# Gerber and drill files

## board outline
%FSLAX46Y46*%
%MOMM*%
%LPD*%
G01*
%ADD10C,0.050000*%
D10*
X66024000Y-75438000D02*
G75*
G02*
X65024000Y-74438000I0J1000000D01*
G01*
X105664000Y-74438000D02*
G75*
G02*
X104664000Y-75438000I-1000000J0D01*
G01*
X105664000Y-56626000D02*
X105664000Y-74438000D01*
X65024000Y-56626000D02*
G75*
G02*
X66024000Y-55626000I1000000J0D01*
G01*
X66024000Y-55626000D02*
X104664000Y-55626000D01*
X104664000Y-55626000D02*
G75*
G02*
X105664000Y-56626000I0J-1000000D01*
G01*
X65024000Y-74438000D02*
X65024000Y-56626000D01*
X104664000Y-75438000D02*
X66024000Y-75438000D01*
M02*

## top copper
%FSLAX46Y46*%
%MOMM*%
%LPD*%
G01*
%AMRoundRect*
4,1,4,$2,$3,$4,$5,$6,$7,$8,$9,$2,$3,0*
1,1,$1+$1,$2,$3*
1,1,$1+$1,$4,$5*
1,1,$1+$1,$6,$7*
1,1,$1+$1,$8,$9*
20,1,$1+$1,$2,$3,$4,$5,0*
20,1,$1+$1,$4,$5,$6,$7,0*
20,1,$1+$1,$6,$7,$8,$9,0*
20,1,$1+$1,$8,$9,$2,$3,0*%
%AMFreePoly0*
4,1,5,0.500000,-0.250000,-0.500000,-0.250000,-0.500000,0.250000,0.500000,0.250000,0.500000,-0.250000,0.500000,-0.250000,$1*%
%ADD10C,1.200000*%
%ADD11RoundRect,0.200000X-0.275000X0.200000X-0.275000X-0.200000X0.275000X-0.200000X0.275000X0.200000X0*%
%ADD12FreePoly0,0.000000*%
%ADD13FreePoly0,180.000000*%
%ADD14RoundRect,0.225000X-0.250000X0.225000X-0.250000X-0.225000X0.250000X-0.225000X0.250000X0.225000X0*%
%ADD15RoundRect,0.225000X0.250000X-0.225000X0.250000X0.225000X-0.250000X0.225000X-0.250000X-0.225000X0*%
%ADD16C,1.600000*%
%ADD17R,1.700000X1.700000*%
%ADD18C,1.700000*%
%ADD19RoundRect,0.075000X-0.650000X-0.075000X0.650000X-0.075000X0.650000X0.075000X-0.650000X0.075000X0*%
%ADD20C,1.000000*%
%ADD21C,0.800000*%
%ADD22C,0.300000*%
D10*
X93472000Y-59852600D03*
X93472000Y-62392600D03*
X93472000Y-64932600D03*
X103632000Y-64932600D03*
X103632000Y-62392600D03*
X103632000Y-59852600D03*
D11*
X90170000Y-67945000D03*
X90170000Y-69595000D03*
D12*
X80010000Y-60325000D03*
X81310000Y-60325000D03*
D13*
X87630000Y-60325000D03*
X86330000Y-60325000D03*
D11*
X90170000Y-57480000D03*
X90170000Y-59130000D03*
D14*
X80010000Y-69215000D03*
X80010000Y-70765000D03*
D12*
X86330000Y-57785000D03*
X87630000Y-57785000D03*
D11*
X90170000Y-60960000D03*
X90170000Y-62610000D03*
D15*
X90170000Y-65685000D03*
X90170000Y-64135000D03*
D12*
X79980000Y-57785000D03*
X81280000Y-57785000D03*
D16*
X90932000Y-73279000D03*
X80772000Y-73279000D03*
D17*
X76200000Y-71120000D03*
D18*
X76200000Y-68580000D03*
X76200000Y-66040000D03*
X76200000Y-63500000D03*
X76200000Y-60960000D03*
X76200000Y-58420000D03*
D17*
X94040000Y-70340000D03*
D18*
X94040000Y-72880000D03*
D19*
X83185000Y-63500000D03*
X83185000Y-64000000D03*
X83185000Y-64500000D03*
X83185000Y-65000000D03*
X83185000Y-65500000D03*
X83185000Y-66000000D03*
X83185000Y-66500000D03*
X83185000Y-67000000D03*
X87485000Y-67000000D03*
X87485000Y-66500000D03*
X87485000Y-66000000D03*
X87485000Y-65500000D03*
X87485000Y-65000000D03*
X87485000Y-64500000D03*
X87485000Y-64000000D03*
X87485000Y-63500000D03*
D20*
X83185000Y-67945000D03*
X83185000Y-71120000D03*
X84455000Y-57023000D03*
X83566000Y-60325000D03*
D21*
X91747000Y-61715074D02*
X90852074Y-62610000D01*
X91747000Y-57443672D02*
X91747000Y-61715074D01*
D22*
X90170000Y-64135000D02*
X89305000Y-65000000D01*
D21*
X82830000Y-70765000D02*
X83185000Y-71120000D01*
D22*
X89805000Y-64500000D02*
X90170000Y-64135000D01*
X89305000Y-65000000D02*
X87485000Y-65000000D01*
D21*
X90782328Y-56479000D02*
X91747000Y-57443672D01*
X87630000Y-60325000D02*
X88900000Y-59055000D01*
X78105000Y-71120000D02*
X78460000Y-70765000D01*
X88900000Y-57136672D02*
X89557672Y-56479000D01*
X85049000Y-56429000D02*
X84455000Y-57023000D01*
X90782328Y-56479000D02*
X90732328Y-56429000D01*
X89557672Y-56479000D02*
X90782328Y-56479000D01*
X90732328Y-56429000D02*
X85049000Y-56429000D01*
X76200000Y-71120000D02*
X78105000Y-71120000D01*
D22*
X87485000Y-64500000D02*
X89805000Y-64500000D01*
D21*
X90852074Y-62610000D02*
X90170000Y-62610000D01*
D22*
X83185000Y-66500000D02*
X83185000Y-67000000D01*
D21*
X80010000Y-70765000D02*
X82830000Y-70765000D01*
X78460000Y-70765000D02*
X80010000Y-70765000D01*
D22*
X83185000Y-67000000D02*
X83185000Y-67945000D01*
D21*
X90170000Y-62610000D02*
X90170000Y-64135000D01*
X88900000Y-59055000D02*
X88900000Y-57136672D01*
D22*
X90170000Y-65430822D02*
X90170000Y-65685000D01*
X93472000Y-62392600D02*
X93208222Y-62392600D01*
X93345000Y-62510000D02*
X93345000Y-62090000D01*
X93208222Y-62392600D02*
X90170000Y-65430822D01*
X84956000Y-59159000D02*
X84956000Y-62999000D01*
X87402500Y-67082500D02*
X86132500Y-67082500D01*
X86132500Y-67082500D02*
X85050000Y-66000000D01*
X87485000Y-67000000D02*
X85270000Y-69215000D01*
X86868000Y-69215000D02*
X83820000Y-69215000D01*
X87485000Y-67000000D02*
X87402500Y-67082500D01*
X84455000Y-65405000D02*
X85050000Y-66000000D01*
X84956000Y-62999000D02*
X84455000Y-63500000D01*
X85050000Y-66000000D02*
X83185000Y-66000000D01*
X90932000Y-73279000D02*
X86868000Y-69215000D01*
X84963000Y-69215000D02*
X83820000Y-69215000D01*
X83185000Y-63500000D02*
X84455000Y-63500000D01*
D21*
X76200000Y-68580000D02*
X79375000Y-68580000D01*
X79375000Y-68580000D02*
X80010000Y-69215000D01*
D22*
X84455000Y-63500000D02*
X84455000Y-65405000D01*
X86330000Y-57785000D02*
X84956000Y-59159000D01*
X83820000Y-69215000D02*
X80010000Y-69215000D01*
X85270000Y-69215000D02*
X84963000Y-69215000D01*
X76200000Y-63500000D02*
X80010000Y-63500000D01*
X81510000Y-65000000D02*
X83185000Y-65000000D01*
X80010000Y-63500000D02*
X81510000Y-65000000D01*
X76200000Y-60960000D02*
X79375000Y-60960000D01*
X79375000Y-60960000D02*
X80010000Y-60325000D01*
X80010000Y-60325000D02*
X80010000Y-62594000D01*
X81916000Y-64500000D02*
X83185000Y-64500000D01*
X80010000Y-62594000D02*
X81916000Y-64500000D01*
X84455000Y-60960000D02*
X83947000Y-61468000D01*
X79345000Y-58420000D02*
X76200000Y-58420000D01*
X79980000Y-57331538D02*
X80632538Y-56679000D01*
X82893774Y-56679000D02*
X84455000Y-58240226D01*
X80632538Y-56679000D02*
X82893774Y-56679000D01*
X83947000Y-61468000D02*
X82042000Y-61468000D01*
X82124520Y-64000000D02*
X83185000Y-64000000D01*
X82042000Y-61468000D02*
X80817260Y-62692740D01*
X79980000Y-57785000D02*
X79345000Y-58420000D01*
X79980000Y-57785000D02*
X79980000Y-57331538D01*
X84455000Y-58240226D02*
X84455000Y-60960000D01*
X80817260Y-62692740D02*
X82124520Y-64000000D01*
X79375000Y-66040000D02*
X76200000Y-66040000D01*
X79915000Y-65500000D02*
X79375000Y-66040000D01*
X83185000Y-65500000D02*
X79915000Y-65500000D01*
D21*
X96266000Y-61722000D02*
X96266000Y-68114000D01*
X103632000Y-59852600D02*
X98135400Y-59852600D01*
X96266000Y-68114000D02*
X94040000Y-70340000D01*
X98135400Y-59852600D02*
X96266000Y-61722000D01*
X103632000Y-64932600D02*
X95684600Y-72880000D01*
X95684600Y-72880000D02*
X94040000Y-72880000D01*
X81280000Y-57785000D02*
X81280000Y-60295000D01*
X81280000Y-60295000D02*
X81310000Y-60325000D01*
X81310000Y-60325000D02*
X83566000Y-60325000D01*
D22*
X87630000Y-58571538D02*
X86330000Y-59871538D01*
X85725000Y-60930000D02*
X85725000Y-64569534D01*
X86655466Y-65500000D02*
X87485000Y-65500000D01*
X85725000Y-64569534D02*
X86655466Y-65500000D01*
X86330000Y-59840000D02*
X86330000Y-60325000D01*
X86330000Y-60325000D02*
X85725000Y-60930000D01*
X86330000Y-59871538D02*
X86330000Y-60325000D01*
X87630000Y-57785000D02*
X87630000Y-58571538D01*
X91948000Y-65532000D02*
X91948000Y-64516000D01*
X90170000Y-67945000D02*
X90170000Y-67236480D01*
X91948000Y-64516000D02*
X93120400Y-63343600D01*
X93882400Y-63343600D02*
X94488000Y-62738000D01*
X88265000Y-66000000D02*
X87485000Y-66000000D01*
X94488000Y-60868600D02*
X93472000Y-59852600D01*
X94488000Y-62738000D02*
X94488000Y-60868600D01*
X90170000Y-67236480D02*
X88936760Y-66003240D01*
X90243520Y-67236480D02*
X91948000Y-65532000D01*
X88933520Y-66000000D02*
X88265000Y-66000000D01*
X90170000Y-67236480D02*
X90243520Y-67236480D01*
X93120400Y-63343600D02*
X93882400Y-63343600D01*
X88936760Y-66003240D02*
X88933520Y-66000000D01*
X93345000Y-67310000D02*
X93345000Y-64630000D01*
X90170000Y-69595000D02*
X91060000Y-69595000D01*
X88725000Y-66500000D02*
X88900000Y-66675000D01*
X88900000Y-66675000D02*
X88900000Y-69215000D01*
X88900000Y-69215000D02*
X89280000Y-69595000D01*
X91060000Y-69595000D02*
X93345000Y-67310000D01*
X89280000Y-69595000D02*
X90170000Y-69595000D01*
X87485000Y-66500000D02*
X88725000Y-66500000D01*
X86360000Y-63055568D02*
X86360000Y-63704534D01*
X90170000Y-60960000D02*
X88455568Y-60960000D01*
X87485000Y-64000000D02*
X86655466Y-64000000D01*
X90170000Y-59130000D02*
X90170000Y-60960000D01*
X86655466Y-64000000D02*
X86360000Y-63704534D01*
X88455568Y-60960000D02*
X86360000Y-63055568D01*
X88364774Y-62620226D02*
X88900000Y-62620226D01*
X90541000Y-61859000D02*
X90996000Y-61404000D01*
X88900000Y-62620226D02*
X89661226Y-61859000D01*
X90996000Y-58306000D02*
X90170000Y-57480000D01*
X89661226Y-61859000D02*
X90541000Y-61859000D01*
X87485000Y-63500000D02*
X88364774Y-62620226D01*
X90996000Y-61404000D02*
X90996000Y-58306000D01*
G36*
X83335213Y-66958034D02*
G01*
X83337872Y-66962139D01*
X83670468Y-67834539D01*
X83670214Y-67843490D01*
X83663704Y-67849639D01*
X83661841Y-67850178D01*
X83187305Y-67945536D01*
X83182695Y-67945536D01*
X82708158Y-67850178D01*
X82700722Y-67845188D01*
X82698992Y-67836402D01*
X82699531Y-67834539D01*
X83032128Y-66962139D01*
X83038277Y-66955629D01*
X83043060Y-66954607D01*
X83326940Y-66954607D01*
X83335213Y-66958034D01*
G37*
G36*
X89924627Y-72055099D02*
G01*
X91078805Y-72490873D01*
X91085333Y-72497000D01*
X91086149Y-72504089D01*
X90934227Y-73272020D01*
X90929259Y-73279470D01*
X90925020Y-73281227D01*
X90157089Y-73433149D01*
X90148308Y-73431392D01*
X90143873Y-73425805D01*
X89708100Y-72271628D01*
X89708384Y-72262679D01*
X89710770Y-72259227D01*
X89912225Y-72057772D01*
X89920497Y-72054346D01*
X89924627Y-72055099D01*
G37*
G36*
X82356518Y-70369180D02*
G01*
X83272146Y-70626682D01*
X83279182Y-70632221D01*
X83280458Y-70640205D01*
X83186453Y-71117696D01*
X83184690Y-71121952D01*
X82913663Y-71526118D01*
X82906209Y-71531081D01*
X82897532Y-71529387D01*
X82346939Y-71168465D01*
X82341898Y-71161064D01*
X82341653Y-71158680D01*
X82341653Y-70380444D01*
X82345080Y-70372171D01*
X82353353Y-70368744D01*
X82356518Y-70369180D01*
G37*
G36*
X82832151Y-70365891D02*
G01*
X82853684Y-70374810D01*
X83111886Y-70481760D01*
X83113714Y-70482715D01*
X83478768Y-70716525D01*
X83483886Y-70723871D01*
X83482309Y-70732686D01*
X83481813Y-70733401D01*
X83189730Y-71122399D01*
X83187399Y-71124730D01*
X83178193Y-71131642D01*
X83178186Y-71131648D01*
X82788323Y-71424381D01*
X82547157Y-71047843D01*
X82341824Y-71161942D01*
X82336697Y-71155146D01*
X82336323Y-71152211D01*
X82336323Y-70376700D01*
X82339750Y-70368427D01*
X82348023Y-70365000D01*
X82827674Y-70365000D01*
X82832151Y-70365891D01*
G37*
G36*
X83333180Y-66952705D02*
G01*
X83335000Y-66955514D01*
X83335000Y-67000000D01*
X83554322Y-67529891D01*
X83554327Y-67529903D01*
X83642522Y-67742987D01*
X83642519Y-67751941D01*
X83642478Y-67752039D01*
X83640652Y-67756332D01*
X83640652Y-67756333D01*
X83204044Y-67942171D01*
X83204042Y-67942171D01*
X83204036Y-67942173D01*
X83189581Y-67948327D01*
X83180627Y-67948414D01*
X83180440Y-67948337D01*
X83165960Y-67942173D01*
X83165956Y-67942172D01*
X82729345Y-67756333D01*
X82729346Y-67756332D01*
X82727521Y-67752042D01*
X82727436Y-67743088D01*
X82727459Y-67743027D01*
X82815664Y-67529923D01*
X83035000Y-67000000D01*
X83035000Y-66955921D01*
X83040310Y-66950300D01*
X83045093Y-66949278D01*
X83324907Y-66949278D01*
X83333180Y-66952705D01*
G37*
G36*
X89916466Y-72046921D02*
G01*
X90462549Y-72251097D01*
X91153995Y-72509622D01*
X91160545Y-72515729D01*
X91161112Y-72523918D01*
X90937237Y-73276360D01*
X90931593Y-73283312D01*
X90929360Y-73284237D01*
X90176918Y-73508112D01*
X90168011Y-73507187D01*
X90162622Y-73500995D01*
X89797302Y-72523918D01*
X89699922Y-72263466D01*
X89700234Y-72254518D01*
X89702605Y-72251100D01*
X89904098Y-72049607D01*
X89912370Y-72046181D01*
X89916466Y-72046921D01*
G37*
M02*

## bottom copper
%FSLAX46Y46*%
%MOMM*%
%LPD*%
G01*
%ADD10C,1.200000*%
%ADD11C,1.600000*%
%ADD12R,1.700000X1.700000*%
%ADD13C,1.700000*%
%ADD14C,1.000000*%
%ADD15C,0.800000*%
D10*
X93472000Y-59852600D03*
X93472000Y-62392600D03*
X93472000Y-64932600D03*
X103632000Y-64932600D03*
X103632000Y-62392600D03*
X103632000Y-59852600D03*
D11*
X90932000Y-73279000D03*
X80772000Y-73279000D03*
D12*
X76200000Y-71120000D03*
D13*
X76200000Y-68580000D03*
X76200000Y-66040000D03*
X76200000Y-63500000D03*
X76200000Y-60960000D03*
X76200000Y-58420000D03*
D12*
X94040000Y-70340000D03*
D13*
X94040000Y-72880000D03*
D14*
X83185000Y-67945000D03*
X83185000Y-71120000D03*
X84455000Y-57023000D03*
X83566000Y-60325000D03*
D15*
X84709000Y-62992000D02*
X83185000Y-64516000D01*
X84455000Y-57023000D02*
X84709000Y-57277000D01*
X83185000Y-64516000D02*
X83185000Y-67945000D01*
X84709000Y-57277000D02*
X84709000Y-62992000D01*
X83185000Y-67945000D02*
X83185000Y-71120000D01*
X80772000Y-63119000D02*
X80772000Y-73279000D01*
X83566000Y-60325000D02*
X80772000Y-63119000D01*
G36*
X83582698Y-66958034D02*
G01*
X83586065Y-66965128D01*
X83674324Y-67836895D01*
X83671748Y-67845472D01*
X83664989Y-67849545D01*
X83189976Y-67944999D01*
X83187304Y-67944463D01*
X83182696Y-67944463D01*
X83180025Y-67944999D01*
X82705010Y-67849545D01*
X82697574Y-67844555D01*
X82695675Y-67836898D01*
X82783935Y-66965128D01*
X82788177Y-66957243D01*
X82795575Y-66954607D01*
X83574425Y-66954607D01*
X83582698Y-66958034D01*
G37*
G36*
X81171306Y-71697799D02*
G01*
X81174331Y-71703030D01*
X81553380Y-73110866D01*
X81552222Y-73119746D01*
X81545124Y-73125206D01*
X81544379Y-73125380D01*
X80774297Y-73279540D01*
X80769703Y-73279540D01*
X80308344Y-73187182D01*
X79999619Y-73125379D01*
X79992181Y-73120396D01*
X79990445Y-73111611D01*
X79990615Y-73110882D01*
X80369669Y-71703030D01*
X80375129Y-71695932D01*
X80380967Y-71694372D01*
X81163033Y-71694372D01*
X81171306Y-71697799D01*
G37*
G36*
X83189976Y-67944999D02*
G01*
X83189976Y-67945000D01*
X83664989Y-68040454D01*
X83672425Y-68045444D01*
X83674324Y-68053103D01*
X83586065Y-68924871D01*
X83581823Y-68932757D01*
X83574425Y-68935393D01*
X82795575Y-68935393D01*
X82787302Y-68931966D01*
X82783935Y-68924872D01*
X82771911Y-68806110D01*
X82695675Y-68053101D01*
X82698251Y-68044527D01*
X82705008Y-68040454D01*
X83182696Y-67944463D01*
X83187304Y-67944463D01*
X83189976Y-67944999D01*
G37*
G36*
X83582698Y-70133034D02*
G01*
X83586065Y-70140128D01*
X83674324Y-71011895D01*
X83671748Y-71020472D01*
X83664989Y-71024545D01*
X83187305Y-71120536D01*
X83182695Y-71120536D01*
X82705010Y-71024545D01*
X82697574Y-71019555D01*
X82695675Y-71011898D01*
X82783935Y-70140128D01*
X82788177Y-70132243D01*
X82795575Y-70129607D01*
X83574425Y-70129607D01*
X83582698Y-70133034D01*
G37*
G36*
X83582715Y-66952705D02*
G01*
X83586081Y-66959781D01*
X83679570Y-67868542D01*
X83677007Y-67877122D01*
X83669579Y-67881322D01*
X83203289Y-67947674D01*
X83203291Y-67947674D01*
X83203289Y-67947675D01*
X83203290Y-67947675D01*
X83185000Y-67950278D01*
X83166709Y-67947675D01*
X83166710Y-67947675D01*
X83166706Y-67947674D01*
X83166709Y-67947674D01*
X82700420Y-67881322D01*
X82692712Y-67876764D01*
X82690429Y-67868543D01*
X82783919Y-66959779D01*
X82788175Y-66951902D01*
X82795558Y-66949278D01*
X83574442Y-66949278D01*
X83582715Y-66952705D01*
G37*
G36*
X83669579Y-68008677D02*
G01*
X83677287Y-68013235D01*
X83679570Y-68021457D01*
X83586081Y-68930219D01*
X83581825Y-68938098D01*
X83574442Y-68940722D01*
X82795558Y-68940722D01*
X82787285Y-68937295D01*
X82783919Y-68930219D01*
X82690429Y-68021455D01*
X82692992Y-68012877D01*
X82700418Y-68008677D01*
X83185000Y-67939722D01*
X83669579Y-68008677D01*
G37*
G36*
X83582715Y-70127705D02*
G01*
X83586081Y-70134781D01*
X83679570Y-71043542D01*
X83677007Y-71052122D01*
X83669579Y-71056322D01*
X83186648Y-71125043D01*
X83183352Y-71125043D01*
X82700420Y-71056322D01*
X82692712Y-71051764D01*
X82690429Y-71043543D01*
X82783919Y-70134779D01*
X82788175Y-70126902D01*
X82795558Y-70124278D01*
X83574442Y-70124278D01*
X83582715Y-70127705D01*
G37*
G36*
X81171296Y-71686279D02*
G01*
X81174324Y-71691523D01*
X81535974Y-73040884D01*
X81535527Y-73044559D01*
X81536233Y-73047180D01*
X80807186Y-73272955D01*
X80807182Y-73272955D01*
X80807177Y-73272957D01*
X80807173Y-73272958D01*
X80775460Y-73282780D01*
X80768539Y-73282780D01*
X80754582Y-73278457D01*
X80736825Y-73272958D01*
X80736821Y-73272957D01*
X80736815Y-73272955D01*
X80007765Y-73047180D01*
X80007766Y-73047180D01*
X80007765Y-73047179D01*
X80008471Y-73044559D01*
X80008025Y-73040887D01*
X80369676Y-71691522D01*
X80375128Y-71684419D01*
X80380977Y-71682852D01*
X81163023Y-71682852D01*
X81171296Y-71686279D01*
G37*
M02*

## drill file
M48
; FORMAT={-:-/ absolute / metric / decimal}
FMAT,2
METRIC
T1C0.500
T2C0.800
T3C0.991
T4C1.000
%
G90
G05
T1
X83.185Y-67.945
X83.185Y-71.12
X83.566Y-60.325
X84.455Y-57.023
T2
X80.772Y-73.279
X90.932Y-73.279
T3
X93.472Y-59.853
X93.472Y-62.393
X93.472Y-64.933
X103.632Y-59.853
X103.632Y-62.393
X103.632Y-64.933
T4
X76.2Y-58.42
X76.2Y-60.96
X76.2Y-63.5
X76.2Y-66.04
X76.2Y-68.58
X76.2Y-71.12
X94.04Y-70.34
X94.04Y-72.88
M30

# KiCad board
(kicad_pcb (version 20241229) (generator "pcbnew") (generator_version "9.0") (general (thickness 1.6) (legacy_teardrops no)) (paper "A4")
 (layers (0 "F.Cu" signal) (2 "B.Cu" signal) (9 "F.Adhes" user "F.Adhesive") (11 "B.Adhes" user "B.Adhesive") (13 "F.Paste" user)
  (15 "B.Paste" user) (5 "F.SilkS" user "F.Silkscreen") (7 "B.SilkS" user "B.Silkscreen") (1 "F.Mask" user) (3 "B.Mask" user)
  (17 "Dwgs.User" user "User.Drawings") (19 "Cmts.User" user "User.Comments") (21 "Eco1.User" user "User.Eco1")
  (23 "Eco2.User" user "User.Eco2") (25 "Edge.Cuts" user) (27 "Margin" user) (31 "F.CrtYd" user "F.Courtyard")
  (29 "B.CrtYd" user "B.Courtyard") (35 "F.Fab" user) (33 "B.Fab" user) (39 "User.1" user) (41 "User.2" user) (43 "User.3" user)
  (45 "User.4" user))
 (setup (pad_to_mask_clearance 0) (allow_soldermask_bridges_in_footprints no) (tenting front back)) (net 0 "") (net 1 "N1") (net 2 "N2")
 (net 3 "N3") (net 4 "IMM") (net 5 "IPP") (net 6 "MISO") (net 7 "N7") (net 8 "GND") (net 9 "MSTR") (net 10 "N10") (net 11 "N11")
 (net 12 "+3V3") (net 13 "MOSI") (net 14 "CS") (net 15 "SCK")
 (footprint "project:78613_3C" (layer "F.Cu") (at 98.552 62.3926)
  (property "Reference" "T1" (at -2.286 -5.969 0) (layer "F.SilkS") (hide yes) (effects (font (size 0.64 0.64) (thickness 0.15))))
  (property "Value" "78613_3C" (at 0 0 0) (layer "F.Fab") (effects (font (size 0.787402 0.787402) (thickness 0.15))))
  (pad "1" thru_hole circle (at -5.08 -2.54) (size 1.2 1.2) (drill 0.9906) (layers "*.Cu" "*.Mask") (remove_unused_layers no) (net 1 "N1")
   (solder_mask_margin 0.102))
  (pad "2" thru_hole circle (at -5.08 0) (size 1.2 1.2) (drill 0.9906) (layers "*.Cu" "*.Mask") (remove_unused_layers no) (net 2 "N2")
   (solder_mask_margin 0.102))
  (pad "3" thru_hole circle (at -5.08 2.54) (size 1.2 1.2) (drill 0.9906) (layers "*.Cu" "*.Mask") (remove_unused_layers no) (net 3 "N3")
   (solder_mask_margin 0.102))
  (pad "4" thru_hole circle (at 5.08 2.54) (size 1.2 1.2) (drill 0.9906) (layers "*.Cu" "*.Mask") (remove_unused_layers no) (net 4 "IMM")
   (solder_mask_margin 0.102))
  (pad "5" thru_hole circle (at 5.08 0) (size 1.2 1.2) (drill 0.9906) (layers "*.Cu" "*.Mask") (remove_unused_layers no)
   (solder_mask_margin 0.102))
  (pad "6" thru_hole circle (at 5.08 -2.54) (size 1.2 1.2) (drill 0.9906) (layers "*.Cu" "*.Mask") (remove_unused_layers no) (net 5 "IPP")
   (solder_mask_margin 0.102)))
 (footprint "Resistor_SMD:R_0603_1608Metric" (layer "F.Cu") (at 90.17 68.77 -90)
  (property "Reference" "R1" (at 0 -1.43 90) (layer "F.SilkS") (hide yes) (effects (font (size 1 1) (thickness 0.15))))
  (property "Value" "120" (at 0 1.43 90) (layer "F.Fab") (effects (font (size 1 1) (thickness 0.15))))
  (pad "1" smd roundrect (at -0.825 0 270) (size 0.8 0.95) (layers "F.Cu" "F.Mask" "F.Paste") (roundrect_rratio 0.25) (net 1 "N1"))
  (pad "2" smd roundrect (at 0.825 0 270) (size 0.8 0.95) (layers "F.Cu" "F.Mask" "F.Paste") (roundrect_rratio 0.25) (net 3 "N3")))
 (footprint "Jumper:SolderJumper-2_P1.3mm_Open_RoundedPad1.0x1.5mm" (layer "F.Cu") (at 80.66 60.325)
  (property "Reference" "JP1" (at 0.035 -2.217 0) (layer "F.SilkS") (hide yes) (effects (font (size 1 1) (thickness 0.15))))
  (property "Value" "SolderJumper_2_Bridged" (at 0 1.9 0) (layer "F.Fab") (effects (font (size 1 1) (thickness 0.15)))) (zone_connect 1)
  (pad "1" smd custom (at -0.65 0) (size 1 0.5) (layers "F.Cu" "F.Mask") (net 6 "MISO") (zone_connect 2) (thermal_bridge_angle 45)
   (options (clearance outline) (anchor rect)) (primitives))
  (pad "2" smd custom (at 0.65 0) (size 1 0.5) (layers "F.Cu" "F.Mask") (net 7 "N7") (zone_connect 2) (thermal_bridge_angle 45)
   (options (clearance outline) (anchor rect)) (primitives)))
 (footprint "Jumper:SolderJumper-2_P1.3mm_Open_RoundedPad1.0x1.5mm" (layer "F.Cu") (at 86.98 60.325 180)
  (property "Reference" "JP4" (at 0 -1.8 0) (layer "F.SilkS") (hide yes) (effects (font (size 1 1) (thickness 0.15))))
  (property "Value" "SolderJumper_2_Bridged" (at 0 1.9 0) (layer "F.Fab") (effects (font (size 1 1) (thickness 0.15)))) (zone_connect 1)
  (pad "1" smd custom (at -0.65 0 180) (size 1 0.5) (layers "F.Cu" "F.Mask") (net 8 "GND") (zone_connect 2) (thermal_bridge_angle 45)
   (options (clearance outline) (anchor rect)) (primitives))
  (pad "2" smd custom (at 0.65 0 180) (size 1 0.5) (layers "F.Cu" "F.Mask") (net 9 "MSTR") (zone_connect 2) (thermal_bridge_angle 45)
   (options (clearance outline) (anchor rect)) (primitives)))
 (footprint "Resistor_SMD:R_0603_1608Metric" (layer "F.Cu") (at 90.17 58.305 -90)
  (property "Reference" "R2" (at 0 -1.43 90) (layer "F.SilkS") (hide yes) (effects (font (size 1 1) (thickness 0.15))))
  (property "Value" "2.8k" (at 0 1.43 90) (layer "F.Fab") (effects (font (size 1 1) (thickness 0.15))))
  (pad "1" smd roundrect (at -0.825 0 270) (size 0.8 0.95) (layers "F.Cu" "F.Mask" "F.Paste") (roundrect_rratio 0.25) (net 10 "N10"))
  (pad "2" smd roundrect (at 0.825 0 270) (size 0.8 0.95) (layers "F.Cu" "F.Mask" "F.Paste") (roundrect_rratio 0.25) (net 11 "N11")))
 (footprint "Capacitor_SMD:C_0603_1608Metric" (layer "F.Cu") (at 80.01 69.99 -90)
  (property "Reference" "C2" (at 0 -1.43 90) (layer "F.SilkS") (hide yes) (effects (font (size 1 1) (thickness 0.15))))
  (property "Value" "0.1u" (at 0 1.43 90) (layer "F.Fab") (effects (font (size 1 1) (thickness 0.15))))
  (pad "1" smd roundrect (at -0.775 0 270) (size 0.9 0.95) (layers "F.Cu" "F.Mask" "F.Paste") (roundrect_rratio 0.25) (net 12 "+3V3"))
  (pad "2" smd roundrect (at 0.775 0 270) (size 0.9 0.95) (layers "F.Cu" "F.Mask" "F.Paste") (roundrect_rratio 0.25) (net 8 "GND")))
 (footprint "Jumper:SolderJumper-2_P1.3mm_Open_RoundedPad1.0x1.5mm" (layer "F.Cu") (at 86.98 57.785)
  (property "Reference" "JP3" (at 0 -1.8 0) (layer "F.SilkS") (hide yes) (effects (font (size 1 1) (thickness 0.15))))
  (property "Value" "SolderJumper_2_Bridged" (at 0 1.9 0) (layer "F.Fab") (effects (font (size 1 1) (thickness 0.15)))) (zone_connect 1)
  (pad "1" smd custom (at -0.65 0) (size 1 0.5) (layers "F.Cu" "F.Mask") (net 12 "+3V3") (zone_connect 2) (thermal_bridge_angle 45)
   (options (clearance outline) (anchor rect)) (primitives))
  (pad "2" smd custom (at 0.65 0) (size 1 0.5) (layers "F.Cu" "F.Mask") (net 9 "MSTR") (zone_connect 2) (thermal_bridge_angle 45)
   (options (clearance outline) (anchor rect)) (primitives)))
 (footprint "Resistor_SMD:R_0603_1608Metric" (layer "F.Cu") (at 90.17 61.785 -90)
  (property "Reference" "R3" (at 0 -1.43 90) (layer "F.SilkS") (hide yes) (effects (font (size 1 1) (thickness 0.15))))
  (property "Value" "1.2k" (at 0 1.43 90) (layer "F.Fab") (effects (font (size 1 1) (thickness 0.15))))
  (pad "1" smd roundrect (at -0.825 0 270) (size 0.8 0.95) (layers "F.Cu" "F.Mask" "F.Paste") (roundrect_rratio 0.25) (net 11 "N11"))
  (pad "2" smd roundrect (at 0.825 0 270) (size 0.8 0.95) (layers "F.Cu" "F.Mask" "F.Paste") (roundrect_rratio 0.25) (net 8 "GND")))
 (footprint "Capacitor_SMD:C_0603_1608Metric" (layer "F.Cu") (at 90.17 64.91 90)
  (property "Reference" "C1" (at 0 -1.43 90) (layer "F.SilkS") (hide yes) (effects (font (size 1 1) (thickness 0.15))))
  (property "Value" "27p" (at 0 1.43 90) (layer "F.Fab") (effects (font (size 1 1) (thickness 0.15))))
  (pad "1" smd roundrect (at -0.775 0 90) (size 0.9 0.95) (layers "F.Cu" "F.Mask" "F.Paste") (roundrect_rratio 0.25) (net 2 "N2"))
  (pad "2" smd roundrect (at 0.775 0 90) (size 0.9 0.95) (layers "F.Cu" "F.Mask" "F.Paste") (roundrect_rratio 0.25) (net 8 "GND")))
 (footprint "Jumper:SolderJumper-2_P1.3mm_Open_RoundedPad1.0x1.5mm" (layer "F.Cu") (at 80.63 57.785)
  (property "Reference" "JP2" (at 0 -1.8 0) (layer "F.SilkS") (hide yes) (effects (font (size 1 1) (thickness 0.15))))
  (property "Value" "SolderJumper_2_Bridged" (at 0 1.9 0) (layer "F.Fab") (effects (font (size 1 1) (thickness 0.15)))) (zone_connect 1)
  (pad "1" smd custom (at -0.65 0) (size 1 0.5) (layers "F.Cu" "F.Mask") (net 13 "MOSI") (zone_connect 2) (thermal_bridge_angle 45)
   (options (clearance outline) (anchor rect)) (primitives))
  (pad "2" smd custom (at 0.65 0) (size 1 0.5) (layers "F.Cu" "F.Mask") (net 7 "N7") (zone_connect 2) (thermal_bridge_angle 45)
   (options (clearance outline) (anchor rect)) (primitives)))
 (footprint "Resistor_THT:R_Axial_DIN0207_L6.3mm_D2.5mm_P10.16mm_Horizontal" (layer "F.Cu") (at 90.932 73.279 180)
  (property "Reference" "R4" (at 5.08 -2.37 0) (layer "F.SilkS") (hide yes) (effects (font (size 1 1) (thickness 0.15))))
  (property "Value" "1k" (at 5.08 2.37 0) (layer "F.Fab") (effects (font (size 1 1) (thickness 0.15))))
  (pad "1" thru_hole circle (at 0 0 180) (size 1.6 1.6) (drill 0.8) (layers "*.Cu" "*.Mask") (remove_unused_layers no) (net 12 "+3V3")
   (teardrops (best_length_ratio 0.5) (max_length 1) (best_width_ratio 1) (max_width 2) (curved_edges no) (filter_ratio 0.9) (enabled yes)
    (allow_two_segments yes) (prefer_zone_connections yes)))
  (pad "2" thru_hole circle (at 10.16 0 180) (size 1.6 1.6) (drill 0.8) (layers "*.Cu" "*.Mask") (remove_unused_layers no) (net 7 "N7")
   (teardrops (best_length_ratio 0.5) (max_length 1) (best_width_ratio 1) (max_width 2) (curved_edges no) (filter_ratio 0.9) (enabled yes)
    (allow_two_segments yes) (prefer_zone_connections yes))))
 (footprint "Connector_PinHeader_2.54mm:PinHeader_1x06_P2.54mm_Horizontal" (layer "F.Cu") (at 76.2 71.12 180)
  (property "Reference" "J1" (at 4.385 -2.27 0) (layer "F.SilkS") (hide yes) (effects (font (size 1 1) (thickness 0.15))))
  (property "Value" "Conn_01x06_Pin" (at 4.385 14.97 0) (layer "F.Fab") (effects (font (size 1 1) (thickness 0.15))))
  (pad "1" thru_hole rect (at 0 0 180) (size 1.7 1.7) (drill 1) (layers "*.Cu" "*.Mask") (remove_unused_layers no) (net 8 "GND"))
  (pad "2" thru_hole circle (at 0 2.54 180) (size 1.7 1.7) (drill 1) (layers "*.Cu" "*.Mask") (remove_unused_layers no) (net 12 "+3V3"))
  (pad "3" thru_hole circle (at 0 5.08 180) (size 1.7 1.7) (drill 1) (layers "*.Cu" "*.Mask") (remove_unused_layers no) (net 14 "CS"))
  (pad "4" thru_hole circle (at 0 7.62 180) (size 1.7 1.7) (drill 1) (layers "*.Cu" "*.Mask") (remove_unused_layers no) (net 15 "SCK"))
  (pad "5" thru_hole circle (at 0 10.16 180) (size 1.7 1.7) (drill 1) (layers "*.Cu" "*.Mask") (remove_unused_layers no) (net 6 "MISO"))
  (pad "6" thru_hole circle (at 0 12.7 180) (size 1.7 1.7) (drill 1) (layers "*.Cu" "*.Mask") (remove_unused_layers no) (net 13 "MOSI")))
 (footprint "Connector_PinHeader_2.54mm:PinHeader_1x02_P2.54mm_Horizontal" (layer "F.Cu") (at 94.04 70.34)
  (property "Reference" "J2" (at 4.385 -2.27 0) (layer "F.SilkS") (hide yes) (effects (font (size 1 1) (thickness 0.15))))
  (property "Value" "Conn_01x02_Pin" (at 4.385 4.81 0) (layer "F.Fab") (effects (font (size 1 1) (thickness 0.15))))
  (pad "1" thru_hole rect (at 0 0) (size 1.7 1.7) (drill 1) (layers "*.Cu" "*.Mask") (remove_unused_layers no) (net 5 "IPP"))
  (pad "2" thru_hole circle (at 0 2.54) (size 1.7 1.7) (drill 1) (layers "*.Cu" "*.Mask") (remove_unused_layers no) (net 4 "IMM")))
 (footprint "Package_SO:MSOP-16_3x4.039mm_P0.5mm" (layer "F.Cu") (at 85.335 65.25)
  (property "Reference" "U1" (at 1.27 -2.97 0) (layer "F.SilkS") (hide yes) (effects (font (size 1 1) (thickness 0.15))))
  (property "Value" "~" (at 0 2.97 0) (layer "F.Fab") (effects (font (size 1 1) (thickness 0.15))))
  (pad "1" smd roundrect (at -2.15 -1.75) (size 1.45 0.3) (layers "F.Cu" "F.Mask" "F.Paste") (roundrect_rratio 0.25) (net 12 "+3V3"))
  (pad "2" smd roundrect (at -2.15 -1.25) (size 1.45 0.3) (layers "F.Cu" "F.Mask" "F.Paste") (roundrect_rratio 0.25) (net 13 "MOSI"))
  (pad "3" smd roundrect (at -2.15 -0.75) (size 1.45 0.3) (layers "F.Cu" "F.Mask" "F.Paste") (roundrect_rratio 0.25) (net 6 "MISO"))
  (pad "4" smd roundrect (at -2.15 -0.25) (size 1.45 0.3) (layers "F.Cu" "F.Mask" "F.Paste") (roundrect_rratio 0.25) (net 15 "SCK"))
  (pad "5" smd roundrect (at -2.15 0.25) (size 1.45 0.3) (layers "F.Cu" "F.Mask" "F.Paste") (roundrect_rratio 0.25) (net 14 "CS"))
  (pad "6" smd roundrect (at -2.15 0.75) (size 1.45 0.3) (layers "F.Cu" "F.Mask" "F.Paste") (roundrect_rratio 0.25) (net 12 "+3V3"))
  (pad "7" smd roundrect (at -2.15 1.25) (size 1.45 0.3) (layers "F.Cu" "F.Mask" "F.Paste") (roundrect_rratio 0.25) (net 8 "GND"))
  (pad "8" smd roundrect (at -2.15 1.75) (size 1.45 0.3) (layers "F.Cu" "F.Mask" "F.Paste") (roundrect_rratio 0.25) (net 8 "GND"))
  (pad "9" smd roundrect (at 2.15 1.75) (size 1.45 0.3) (layers "F.Cu" "F.Mask" "F.Paste") (roundrect_rratio 0.25) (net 12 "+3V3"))
  (pad "10" smd roundrect (at 2.15 1.25) (size 1.45 0.3) (layers "F.Cu" "F.Mask" "F.Paste") (roundrect_rratio 0.25) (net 3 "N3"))
  (pad "11" smd roundrect (at 2.15 0.75) (size 1.45 0.3) (layers "F.Cu" "F.Mask" "F.Paste") (roundrect_rratio 0.25) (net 1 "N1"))
  (pad "12" smd roundrect (at 2.15 0.25) (size 1.45 0.3) (layers "F.Cu" "F.Mask" "F.Paste") (roundrect_rratio 0.25) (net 9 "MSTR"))
  (pad "13" smd roundrect (at 2.15 -0.25) (size 1.45 0.3) (layers "F.Cu" "F.Mask" "F.Paste") (roundrect_rratio 0.25) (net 8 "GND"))
  (pad "14" smd roundrect (at 2.15 -0.75) (size 1.45 0.3) (layers "F.Cu" "F.Mask" "F.Paste") (roundrect_rratio 0.25) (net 8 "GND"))
  (pad "15" smd roundrect (at 2.15 -1.25) (size 1.45 0.3) (layers "F.Cu" "F.Mask" "F.Paste") (roundrect_rratio 0.25) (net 11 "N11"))
  (pad "16" smd roundrect (at 2.15 -1.75) (size 1.45 0.3) (layers "F.Cu" "F.Mask" "F.Paste") (roundrect_rratio 0.25) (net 10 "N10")))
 (gr_arc (start 66.024 75.438) (mid 65.316893 75.145107) (end 65.024 74.438) (stroke (width 0.05) (type default)) (layer "Edge.Cuts"))
 (gr_arc (start 105.664 74.438) (mid 105.371107 75.145107) (end 104.664 75.438) (stroke (width 0.05) (type default)) (layer "Edge.Cuts"))
 (gr_line (start 105.664 56.626) (end 105.664 74.438) (stroke (width 0.05) (type default)) (layer "Edge.Cuts"))
 (gr_arc (start 65.024 56.626) (mid 65.316893 55.918893) (end 66.024 55.626) (stroke (width 0.05) (type default)) (layer "Edge.Cuts"))
 (gr_line (start 66.024 55.626) (end 104.664 55.626) (stroke (width 0.05) (type default)) (layer "Edge.Cuts"))
 (gr_arc (start 104.664 55.626) (mid 105.371107 55.918893) (end 105.664 56.626) (stroke (width 0.05) (type default)) (layer "Edge.Cuts"))
 (gr_line (start 65.024 74.438) (end 65.024 56.626) (stroke (width 0.05) (type default)) (layer "Edge.Cuts"))
 (gr_line (start 104.664 75.438) (end 66.024 75.438) (stroke (width 0.05) (type default)) (layer "Edge.Cuts"))
 (segment (start 91.747 61.715074) (end 90.852074 62.61) (width 0.8) (layer "F.Cu") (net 8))
 (segment (start 91.747 57.443672) (end 91.747 61.715074) (width 0.8) (layer "F.Cu") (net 8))
 (segment (start 90.17 64.135) (end 89.305 65) (width 0.3) (layer "F.Cu") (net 8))
 (segment (start 82.83 70.765) (end 83.185 71.12) (width 0.8) (layer "F.Cu") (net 8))
 (segment (start 89.805 64.5) (end 90.17 64.135) (width 0.3) (layer "F.Cu") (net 8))
 (segment (start 89.305 65) (end 87.485 65) (width 0.3) (layer "F.Cu") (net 8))
 (segment (start 90.782328 56.479) (end 91.747 57.443672) (width 0.8) (layer "F.Cu") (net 8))
 (segment (start 87.63 60.325) (end 88.9 59.055) (width 0.8) (layer "F.Cu") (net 8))
 (segment (start 78.105 71.12) (end 78.46 70.765) (width 0.8) (layer "F.Cu") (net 8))
 (segment (start 88.9 57.136672) (end 89.557672 56.479) (width 0.8) (layer "F.Cu") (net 8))
 (segment (start 85.049 56.429) (end 84.455 57.023) (width 0.8) (layer "F.Cu") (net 8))
 (segment (start 90.782328 56.479) (end 90.732328 56.429) (width 0.8) (layer "F.Cu") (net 8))
 (segment (start 89.557672 56.479) (end 90.782328 56.479) (width 0.8) (layer "F.Cu") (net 8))
 (segment (start 90.732328 56.429) (end 85.049 56.429) (width 0.8) (layer "F.Cu") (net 8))
 (segment (start 76.2 71.12) (end 78.105 71.12) (width 0.8) (layer "F.Cu") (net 8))
 (segment (start 87.485 64.5) (end 89.805 64.5) (width 0.3) (layer "F.Cu") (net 8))
 (segment (start 90.852074 62.61) (end 90.17 62.61) (width 0.8) (layer "F.Cu") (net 8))
 (segment (start 83.185 66.5) (end 83.185 67) (width 0.3) (layer "F.Cu") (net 8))
 (segment (start 80.01 70.765) (end 82.83 70.765) (width 0.8) (layer "F.Cu") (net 8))
 (segment (start 78.46 70.765) (end 80.01 70.765) (width 0.8) (layer "F.Cu") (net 8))
 (segment (start 83.185 67) (end 83.185 67.945) (width 0.3) (layer "F.Cu") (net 8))
 (segment (start 90.17 62.61) (end 90.17 64.135) (width 0.8) (layer "F.Cu") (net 8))
 (segment (start 88.9 59.055) (end 88.9 57.136672) (width 0.8) (layer "F.Cu") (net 8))
 (via (at 83.185 67.945) (size 1) (drill 0.5) (layers "F.Cu" "B.Cu") (free yes)
  (teardrops (best_length_ratio 0.5) (max_length 1) (best_width_ratio 1) (max_width 2) (curved_edges no) (filter_ratio 0.9) (enabled yes)
   (allow_two_segments yes) (prefer_zone_connections yes))
  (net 8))
 (via (at 83.185 71.12) (size 1) (drill 0.5) (layers "F.Cu" "B.Cu") (free yes)
  (teardrops (best_length_ratio 0.5) (max_length 1) (best_width_ratio 1) (max_width 2) (curved_edges no) (filter_ratio 0.9) (enabled yes)
   (allow_two_segments yes) (prefer_zone_connections yes))
  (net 8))
 (via (at 84.455 57.023) (size 1) (drill 0.5) (layers "F.Cu" "B.Cu") (free yes) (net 8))
 (segment (start 84.709 62.992) (end 83.185 64.516) (width 0.8) (layer "B.Cu") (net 8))
 (segment (start 84.455 57.023) (end 84.709 57.277) (width 0.8) (layer "B.Cu") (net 8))
 (segment (start 83.185 64.516) (end 83.185 67.945) (width 0.8) (layer "B.Cu") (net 8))
 (segment (start 84.709 57.277) (end 84.709 62.992) (width 0.8) (layer "B.Cu") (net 8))
 (segment (start 83.185 67.945) (end 83.185 71.12) (width 0.8) (layer "B.Cu") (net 8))
 (segment (start 90.17 65.430822) (end 90.17 65.685) (width 0.3) (layer "F.Cu") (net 2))
 (segment (start 93.472 62.3926) (end 93.208222 62.3926) (width 0.3) (layer "F.Cu") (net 2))
 (segment (start 93.345 62.51) (end 93.345 62.09) (width 0.3) (layer "F.Cu") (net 2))
 (segment (start 93.208222 62.3926) (end 90.17 65.430822) (width 0.3) (layer "F.Cu") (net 2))
 (segment (start 84.956 59.159) (end 84.956 62.999) (width 0.3) (layer "F.Cu") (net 12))
 (segment (start 87.4025 67.0825) (end 86.1325 67.0825) (width 0.3) (layer "F.Cu") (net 12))
 (segment (start 86.1325 67.0825) (end 85.05 66) (width 0.3) (layer "F.Cu") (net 12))
 (segment (start 87.485 67) (end 85.27 69.215) (width 0.3) (layer "F.Cu") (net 12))
 (segment (start 86.868 69.215) (end 83.82 69.215) (width 0.3) (layer "F.Cu") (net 12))
 (segment (start 87.485 67) (end 87.4025 67.0825) (width 0.3) (layer "F.Cu") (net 12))
 (segment (start 84.455 65.405) (end 85.05 66) (width 0.3) (layer "F.Cu") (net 12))
 (segment (start 84.956 62.999) (end 84.455 63.5) (width 0.3) (layer "F.Cu") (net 12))
 (segment (start 85.05 66) (end 83.185 66) (width 0.3) (layer "F.Cu") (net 12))
 (segment (start 90.932 73.279) (end 86.868 69.215) (width 0.3) (layer "F.Cu") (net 12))
 (segment (start 84.963 69.215) (end 83.82 69.215) (width 0.3) (layer "F.Cu") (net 12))
 (segment (start 83.185 63.5) (end 84.455 63.5) (width 0.3) (layer "F.Cu") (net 12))
 (segment (start 76.2 68.58) (end 79.375 68.58) (width 0.8) (layer "F.Cu") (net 12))
 (segment (start 79.375 68.58) (end 80.01 69.215) (width 0.8) (layer "F.Cu") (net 12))
 (segment (start 84.455 63.5) (end 84.455 65.405) (width 0.3) (layer "F.Cu") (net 12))
 (segment (start 86.33 57.785) (end 84.956 59.159) (width 0.3) (layer "F.Cu") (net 12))
 (segment (start 83.82 69.215) (end 80.01 69.215) (width 0.3) (layer "F.Cu") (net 12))
 (segment (start 85.27 69.215) (end 84.963 69.215) (width 0.3) (layer "F.Cu") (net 12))
 (segment (start 76.2 63.5) (end 80.01 63.5) (width 0.3) (layer "F.Cu") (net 15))
 (segment (start 81.51 65) (end 83.185 65) (width 0.3) (layer "F.Cu") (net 15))
 (segment (start 80.01 63.5) (end 81.51 65) (width 0.3) (layer "F.Cu") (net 15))
 (segment (start 76.2 60.96) (end 79.375 60.96) (width 0.3) (layer "F.Cu") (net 6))
 (segment (start 79.375 60.96) (end 80.01 60.325) (width 0.3) (layer "F.Cu") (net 6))
 (segment (start 80.01 60.325) (end 80.01 62.594) (width 0.3) (layer "F.Cu") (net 6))
 (segment (start 81.916 64.5) (end 83.185 64.5) (width 0.3) (layer "F.Cu") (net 6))
 (segment (start 80.01 62.594) (end 81.916 64.5) (width 0.3) (layer "F.Cu") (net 6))
 (segment (start 84.455 60.96) (end 83.947 61.468) (width 0.3) (layer "F.Cu") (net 13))
 (segment (start 79.345 58.42) (end 76.2 58.42) (width 0.3) (layer "F.Cu") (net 13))
 (segment (start 79.98 57.331538) (end 80.632538 56.679) (width 0.3) (layer "F.Cu") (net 13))
 (segment (start 82.893774 56.679) (end 84.455 58.240226) (width 0.3) (layer "F.Cu") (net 13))
 (segment (start 80.632538 56.679) (end 82.893774 56.679) (width 0.3) (layer "F.Cu") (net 13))
 (segment (start 83.947 61.468) (end 82.042 61.468) (width 0.3) (layer "F.Cu") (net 13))
 (segment (start 82.12452 64) (end 83.185 64) (width 0.3) (layer "F.Cu") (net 13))
 (segment (start 82.042 61.468) (end 80.81726 62.69274) (width 0.3) (layer "F.Cu") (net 13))
 (segment (start 79.98 57.785) (end 79.345 58.42) (width 0.3) (layer "F.Cu") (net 13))
 (segment (start 79.98 57.785) (end 79.98 57.331538) (width 0.3) (layer "F.Cu") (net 13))
 (segment (start 84.455 58.240226) (end 84.455 60.96) (width 0.3) (layer "F.Cu") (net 13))
 (segment (start 80.81726 62.69274) (end 82.12452 64) (width 0.3) (layer "F.Cu") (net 13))
 (segment (start 79.375 66.04) (end 76.2 66.04) (width 0.3) (layer "F.Cu") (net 14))
 (segment (start 79.915 65.5) (end 79.375 66.04) (width 0.3) (layer "F.Cu") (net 14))
 (segment (start 83.185 65.5) (end 79.915 65.5) (width 0.3) (layer "F.Cu") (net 14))
 (segment (start 96.266 61.722) (end 96.266 68.114) (width 0.8) (layer "F.Cu") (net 5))
 (segment (start 103.632 59.8526) (end 98.1354 59.8526) (width 0.8) (layer "F.Cu") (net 5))
 (segment (start 96.266 68.114) (end 94.04 70.34) (width 0.8) (layer "F.Cu") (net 5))
 (segment (start 98.1354 59.8526) (end 96.266 61.722) (width 0.8) (layer "F.Cu") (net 5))
 (segment (start 103.632 64.9326) (end 95.6846 72.88) (width 0.8) (layer "F.Cu") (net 4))
 (segment (start 95.6846 72.88) (end 94.04 72.88) (width 0.8) (layer "F.Cu") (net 4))
 (segment (start 81.28 57.785) (end 81.28 60.295) (width 0.8) (layer "F.Cu") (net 7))
 (segment (start 81.28 60.295) (end 81.31 60.325) (width 0.8) (layer "F.Cu") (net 7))
 (segment (start 81.31 60.325) (end 83.566 60.325) (width 0.8) (layer "F.Cu") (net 7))
 (via (at 83.566 60.325) (size 1) (drill 0.5) (layers "F.Cu" "B.Cu") (free yes) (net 7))
 (segment (start 80.772 63.119) (end 80.772 73.279) (width 0.8) (layer "B.Cu") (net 7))
 (segment (start 83.566 60.325) (end 80.772 63.119) (width 0.8) (layer "B.Cu") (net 7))
 (segment (start 87.63 58.571538) (end 86.33 59.871538) (width 0.3) (layer "F.Cu") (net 9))
 (segment (start 85.725 60.93) (end 85.725 64.569534) (width 0.3) (layer "F.Cu") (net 9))
 (segment (start 86.655466 65.5) (end 87.485 65.5) (width 0.3) (layer "F.Cu") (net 9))
 (segment (start 85.725 64.569534) (end 86.655466 65.5) (width 0.3) (layer "F.Cu") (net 9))
 (segment (start 86.33 59.84) (end 86.33 60.325) (width 0.3) (layer "F.Cu") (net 9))
 (segment (start 86.33 60.325) (end 85.725 60.93) (width 0.3) (layer "F.Cu") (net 9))
 (segment (start 86.33 59.871538) (end 86.33 60.325) (width 0.3) (layer "F.Cu") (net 9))
 (segment (start 87.63 57.785) (end 87.63 58.571538) (width 0.3) (layer "F.Cu") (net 9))
 (segment (start 91.948 65.532) (end 91.948 64.516) (width 0.3) (layer "F.Cu") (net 1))
 (segment (start 90.17 67.945) (end 90.17 67.23648) (width 0.3) (layer "F.Cu") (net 1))
 (segment (start 91.948 64.516) (end 93.1204 63.3436) (width 0.3) (layer "F.Cu") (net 1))
 (segment (start 93.8824 63.3436) (end 94.488 62.738) (width 0.3) (layer "F.Cu") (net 1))
 (segment (start 88.265 66) (end 87.485 66) (width 0.3) (layer "F.Cu") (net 1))
 (segment (start 94.488 60.8686) (end 93.472 59.8526) (width 0.3) (layer "F.Cu") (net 1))
 (segment (start 94.488 62.738) (end 94.488 60.8686) (width 0.3) (layer "F.Cu") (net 1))
 (segment (start 90.17 67.23648) (end 88.93676 66.00324) (width 0.3) (layer "F.Cu") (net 1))
 (segment (start 90.24352 67.23648) (end 91.948 65.532) (width 0.3) (layer "F.Cu") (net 1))
 (segment (start 88.93352 66) (end 88.265 66) (width 0.3) (layer "F.Cu") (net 1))
 (segment (start 90.17 67.23648) (end 90.24352 67.23648) (width 0.3) (layer "F.Cu") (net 1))
 (segment (start 93.1204 63.3436) (end 93.8824 63.3436) (width 0.3) (layer "F.Cu") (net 1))
 (segment (start 88.93676 66.00324) (end 88.93352 66) (width 0.3) (layer "F.Cu") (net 1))
 (segment (start 93.345 67.31) (end 93.345 64.63) (width 0.3) (layer "F.Cu") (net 3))
 (segment (start 90.17 69.595) (end 91.06 69.595) (width 0.3) (layer "F.Cu") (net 3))
 (segment (start 88.725 66.5) (end 88.9 66.675) (width 0.3) (layer "F.Cu") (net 3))
 (segment (start 88.9 66.675) (end 88.9 69.215) (width 0.3) (layer "F.Cu") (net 3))
 (segment (start 88.9 69.215) (end 89.28 69.595) (width 0.3) (layer "F.Cu") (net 3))
 (segment (start 91.06 69.595) (end 93.345 67.31) (width 0.3) (layer "F.Cu") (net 3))
 (segment (start 89.28 69.595) (end 90.17 69.595) (width 0.3) (layer "F.Cu") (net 3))
 (segment (start 87.485 66.5) (end 88.725 66.5) (width 0.3) (layer "F.Cu") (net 3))
 (segment (start 86.36 63.055568) (end 86.36 63.704534) (width 0.3) (layer "F.Cu") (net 11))
 (segment (start 90.17 60.96) (end 88.455568 60.96) (width 0.3) (layer "F.Cu") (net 11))
 (segment (start 87.485 64) (end 86.655466 64) (width 0.3) (layer "F.Cu") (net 11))
 (segment (start 90.17 59.13) (end 90.17 60.96) (width 0.3) (layer "F.Cu") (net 11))
 (segment (start 86.655466 64) (end 86.36 63.704534) (width 0.3) (layer "F.Cu") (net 11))
 (segment (start 88.455568 60.96) (end 86.36 63.055568) (width 0.3) (layer "F.Cu") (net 11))
 (segment (start 88.364774 62.620226) (end 88.9 62.620226) (width 0.3) (layer "F.Cu") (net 10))
 (segment (start 90.541 61.859) (end 90.996 61.404) (width 0.3) (layer "F.Cu") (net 10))
 (segment (start 88.9 62.620226) (end 89.661226 61.859) (width 0.3) (layer "F.Cu") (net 10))
 (segment (start 90.996 58.306) (end 90.17 57.48) (width 0.3) (layer "F.Cu") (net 10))
 (segment (start 89.661226 61.859) (end 90.541 61.859) (width 0.3) (layer "F.Cu") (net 10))
 (segment (start 87.485 63.5) (end 88.364774 62.620226) (width 0.3) (layer "F.Cu") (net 10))
 (segment (start 90.996 61.404) (end 90.996 58.306) (width 0.3) (layer "F.Cu") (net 10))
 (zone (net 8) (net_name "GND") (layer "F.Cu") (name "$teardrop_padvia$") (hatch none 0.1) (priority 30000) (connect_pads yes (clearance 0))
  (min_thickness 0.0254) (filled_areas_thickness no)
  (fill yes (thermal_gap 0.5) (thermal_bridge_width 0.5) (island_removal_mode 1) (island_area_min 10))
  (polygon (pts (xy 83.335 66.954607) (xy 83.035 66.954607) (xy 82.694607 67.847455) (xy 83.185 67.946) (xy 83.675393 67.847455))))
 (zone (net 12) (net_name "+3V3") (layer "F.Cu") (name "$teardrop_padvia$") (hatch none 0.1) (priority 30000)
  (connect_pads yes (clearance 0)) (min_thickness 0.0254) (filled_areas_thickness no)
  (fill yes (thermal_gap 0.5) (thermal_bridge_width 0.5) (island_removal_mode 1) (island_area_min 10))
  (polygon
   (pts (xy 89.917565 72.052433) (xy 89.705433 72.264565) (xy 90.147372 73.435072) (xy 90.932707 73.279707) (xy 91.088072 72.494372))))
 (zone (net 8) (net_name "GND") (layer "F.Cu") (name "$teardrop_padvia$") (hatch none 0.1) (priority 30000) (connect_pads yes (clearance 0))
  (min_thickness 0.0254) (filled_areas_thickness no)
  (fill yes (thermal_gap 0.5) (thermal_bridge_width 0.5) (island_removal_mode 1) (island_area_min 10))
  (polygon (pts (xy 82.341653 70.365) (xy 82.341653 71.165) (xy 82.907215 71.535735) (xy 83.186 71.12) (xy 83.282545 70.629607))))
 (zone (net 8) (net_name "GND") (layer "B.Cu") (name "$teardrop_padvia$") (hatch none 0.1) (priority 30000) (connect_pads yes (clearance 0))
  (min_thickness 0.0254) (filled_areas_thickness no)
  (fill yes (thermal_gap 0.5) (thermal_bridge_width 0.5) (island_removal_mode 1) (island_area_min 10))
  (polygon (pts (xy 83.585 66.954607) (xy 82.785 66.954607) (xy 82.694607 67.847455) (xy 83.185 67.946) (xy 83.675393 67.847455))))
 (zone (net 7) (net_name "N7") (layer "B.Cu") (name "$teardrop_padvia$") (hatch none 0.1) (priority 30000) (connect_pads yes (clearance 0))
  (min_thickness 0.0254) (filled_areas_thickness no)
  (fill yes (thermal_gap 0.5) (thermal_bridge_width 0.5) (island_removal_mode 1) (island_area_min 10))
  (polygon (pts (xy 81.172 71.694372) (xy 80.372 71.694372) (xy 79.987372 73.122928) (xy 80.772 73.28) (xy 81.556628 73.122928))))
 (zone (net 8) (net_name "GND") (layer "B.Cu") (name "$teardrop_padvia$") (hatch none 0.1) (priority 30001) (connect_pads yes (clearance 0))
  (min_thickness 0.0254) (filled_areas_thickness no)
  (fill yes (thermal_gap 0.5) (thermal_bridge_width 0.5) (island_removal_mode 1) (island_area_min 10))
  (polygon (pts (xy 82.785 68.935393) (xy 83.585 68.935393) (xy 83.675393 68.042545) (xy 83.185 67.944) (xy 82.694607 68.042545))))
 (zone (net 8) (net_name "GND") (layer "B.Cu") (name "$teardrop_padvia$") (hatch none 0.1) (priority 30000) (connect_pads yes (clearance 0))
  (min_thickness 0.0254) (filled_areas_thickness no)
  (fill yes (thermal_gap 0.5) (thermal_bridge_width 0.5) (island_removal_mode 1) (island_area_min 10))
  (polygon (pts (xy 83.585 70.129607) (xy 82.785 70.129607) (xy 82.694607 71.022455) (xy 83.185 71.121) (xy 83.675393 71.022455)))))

